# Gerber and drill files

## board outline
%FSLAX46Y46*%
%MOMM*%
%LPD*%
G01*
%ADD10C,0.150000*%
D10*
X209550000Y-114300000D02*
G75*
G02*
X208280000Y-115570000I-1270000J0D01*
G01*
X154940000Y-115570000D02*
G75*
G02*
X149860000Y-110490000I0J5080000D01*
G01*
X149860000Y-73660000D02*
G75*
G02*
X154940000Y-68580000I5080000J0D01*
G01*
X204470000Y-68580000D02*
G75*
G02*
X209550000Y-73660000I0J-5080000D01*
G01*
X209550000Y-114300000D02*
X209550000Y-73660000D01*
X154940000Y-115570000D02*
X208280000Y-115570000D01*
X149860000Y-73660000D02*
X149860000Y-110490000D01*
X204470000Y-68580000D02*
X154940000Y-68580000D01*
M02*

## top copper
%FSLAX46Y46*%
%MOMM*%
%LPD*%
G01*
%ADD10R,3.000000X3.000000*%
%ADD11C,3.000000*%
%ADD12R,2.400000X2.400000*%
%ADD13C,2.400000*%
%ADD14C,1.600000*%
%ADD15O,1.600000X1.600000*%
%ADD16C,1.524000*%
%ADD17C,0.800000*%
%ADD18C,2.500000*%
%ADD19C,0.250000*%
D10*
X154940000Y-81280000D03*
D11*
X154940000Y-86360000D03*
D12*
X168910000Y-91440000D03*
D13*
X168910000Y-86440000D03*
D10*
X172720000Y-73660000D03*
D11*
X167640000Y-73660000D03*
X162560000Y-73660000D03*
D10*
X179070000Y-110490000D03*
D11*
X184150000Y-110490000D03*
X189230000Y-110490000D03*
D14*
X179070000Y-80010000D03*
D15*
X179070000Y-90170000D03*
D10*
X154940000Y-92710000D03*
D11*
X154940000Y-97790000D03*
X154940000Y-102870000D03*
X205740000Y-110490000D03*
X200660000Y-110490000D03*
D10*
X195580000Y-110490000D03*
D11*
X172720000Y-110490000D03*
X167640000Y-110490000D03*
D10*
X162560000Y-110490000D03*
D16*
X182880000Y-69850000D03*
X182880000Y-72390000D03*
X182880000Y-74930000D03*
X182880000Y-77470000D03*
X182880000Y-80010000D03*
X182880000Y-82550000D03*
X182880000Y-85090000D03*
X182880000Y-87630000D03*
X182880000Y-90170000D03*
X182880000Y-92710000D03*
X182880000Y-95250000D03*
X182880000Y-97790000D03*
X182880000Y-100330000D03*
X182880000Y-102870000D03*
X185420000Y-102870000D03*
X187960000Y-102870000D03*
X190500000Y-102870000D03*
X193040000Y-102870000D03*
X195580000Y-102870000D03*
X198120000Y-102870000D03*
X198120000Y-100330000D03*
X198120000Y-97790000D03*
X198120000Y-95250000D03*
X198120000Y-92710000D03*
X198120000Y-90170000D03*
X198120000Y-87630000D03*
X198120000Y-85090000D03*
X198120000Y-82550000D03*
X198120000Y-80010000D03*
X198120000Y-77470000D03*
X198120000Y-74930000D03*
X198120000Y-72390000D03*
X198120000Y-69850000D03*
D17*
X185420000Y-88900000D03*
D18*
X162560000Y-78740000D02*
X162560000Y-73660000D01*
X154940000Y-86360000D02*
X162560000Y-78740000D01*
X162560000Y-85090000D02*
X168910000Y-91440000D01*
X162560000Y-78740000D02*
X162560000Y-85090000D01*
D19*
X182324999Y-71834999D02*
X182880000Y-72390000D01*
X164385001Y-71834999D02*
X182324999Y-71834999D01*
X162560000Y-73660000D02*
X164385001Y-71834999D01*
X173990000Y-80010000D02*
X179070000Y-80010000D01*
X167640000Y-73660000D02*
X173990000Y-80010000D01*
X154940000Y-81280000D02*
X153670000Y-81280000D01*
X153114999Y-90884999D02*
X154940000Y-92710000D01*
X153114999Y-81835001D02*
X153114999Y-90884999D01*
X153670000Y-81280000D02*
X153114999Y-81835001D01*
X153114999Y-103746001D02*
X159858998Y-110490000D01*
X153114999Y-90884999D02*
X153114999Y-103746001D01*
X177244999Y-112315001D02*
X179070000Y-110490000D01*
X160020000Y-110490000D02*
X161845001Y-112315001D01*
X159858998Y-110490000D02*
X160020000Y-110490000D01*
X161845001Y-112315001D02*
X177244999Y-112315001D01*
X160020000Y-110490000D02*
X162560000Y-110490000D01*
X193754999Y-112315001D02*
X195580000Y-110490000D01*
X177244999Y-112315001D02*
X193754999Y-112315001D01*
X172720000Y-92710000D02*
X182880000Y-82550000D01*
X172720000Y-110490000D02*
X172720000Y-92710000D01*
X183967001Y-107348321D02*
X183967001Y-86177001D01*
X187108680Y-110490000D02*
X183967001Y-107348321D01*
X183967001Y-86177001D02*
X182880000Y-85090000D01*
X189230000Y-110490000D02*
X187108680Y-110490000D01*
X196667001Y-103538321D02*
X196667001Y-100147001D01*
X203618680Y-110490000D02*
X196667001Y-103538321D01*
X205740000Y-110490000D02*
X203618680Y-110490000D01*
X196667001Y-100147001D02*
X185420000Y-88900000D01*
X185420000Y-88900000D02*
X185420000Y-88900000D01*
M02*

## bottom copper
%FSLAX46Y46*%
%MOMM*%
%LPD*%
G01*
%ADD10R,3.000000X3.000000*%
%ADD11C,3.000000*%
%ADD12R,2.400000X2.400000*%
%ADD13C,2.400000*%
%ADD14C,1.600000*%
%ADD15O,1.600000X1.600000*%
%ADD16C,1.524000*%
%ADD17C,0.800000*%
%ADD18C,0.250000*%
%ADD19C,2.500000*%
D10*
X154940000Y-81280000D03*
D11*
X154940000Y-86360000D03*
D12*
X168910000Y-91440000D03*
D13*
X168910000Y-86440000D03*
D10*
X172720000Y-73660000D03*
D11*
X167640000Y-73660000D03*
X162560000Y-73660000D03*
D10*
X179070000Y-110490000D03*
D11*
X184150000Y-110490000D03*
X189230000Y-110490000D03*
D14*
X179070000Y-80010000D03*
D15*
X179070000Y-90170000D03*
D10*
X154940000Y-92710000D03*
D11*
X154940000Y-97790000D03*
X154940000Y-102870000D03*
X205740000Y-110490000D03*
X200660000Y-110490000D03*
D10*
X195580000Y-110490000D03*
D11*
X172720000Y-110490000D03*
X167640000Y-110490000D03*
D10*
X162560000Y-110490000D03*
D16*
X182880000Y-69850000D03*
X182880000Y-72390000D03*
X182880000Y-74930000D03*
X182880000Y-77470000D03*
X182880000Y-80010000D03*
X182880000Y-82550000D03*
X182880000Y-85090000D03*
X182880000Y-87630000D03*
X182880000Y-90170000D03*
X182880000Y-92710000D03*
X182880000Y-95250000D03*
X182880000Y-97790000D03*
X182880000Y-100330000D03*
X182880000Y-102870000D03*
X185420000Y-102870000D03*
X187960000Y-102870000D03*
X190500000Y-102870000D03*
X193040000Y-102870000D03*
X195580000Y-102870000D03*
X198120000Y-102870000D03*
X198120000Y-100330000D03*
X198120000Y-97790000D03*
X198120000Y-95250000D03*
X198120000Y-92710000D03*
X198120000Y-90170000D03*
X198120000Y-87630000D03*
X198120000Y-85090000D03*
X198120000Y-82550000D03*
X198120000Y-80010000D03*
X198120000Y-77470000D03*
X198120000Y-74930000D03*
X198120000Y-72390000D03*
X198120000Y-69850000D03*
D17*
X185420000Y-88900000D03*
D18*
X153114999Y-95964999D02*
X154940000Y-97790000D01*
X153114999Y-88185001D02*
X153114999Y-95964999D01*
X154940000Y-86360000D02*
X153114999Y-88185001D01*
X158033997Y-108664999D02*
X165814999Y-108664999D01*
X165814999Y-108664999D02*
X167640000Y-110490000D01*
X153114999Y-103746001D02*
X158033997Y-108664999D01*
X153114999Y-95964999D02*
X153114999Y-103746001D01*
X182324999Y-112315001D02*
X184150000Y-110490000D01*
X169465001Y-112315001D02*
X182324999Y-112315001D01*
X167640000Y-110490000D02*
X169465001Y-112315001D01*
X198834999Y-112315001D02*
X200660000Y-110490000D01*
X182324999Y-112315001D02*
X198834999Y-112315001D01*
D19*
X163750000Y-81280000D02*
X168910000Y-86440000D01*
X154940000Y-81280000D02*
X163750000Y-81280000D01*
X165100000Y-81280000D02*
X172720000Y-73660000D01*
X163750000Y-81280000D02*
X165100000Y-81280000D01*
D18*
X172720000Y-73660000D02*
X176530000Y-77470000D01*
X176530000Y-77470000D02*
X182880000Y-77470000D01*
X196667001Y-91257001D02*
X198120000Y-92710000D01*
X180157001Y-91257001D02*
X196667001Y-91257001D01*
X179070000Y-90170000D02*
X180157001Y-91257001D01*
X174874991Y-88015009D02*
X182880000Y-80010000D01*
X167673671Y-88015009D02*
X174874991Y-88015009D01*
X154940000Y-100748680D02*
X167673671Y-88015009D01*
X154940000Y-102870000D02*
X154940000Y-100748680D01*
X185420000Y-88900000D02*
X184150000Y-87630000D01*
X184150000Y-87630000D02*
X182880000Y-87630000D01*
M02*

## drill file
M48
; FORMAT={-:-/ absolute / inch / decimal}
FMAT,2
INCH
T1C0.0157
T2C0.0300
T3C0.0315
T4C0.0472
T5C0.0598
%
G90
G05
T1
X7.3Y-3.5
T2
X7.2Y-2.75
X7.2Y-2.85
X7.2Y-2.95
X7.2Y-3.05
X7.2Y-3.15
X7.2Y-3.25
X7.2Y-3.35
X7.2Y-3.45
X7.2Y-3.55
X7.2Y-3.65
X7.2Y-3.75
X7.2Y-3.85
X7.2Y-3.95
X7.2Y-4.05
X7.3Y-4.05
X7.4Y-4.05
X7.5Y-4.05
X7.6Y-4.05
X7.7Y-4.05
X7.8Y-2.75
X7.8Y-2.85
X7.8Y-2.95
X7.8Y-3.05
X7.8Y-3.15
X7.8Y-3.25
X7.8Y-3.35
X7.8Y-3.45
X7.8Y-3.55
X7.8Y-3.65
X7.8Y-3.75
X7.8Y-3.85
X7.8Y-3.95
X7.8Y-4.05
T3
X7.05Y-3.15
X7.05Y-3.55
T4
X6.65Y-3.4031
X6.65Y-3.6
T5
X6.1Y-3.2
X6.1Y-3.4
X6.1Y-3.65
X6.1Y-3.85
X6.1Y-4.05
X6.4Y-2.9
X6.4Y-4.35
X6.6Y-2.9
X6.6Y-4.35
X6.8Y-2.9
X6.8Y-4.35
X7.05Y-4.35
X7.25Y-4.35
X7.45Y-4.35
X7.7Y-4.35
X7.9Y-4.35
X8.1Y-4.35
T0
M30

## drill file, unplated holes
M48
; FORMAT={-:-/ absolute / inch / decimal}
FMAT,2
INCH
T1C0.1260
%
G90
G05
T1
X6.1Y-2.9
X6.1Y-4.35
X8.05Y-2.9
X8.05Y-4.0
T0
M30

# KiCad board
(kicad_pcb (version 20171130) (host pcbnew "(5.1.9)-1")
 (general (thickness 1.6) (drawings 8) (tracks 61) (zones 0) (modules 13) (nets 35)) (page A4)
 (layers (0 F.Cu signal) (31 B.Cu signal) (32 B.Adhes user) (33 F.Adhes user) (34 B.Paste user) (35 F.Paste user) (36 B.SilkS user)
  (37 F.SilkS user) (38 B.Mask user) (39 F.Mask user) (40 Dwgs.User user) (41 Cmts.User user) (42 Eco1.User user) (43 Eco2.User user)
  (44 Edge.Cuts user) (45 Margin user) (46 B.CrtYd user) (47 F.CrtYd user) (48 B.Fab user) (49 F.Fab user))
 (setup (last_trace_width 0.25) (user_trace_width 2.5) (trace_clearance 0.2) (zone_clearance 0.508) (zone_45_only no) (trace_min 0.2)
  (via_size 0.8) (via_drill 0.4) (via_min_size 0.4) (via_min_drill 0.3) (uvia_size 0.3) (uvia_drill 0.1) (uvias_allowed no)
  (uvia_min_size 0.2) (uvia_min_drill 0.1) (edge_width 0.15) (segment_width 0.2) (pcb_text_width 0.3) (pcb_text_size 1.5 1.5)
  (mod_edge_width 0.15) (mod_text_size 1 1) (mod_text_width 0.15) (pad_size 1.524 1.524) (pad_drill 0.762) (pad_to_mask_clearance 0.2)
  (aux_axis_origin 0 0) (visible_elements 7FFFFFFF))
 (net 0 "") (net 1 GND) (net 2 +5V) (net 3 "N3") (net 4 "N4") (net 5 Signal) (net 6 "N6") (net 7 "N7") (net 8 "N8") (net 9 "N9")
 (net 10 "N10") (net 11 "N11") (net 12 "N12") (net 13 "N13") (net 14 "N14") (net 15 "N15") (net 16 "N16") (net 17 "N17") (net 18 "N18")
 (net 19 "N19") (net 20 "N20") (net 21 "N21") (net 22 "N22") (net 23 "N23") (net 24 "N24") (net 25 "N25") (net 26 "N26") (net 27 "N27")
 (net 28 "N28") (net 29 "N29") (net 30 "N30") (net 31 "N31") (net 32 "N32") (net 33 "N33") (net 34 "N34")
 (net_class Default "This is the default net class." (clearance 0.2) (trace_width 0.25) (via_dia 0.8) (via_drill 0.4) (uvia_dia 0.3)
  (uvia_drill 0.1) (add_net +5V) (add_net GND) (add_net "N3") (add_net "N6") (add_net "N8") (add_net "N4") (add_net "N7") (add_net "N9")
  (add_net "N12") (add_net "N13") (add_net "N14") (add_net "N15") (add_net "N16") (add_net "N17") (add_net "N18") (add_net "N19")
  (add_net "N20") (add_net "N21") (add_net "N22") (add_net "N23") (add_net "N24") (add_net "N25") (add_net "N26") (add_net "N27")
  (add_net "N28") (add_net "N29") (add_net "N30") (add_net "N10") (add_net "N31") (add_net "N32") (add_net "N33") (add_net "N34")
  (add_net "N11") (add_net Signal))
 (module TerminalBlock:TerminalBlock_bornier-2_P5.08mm (layer F.Cu) (at 154.94 81.28 270)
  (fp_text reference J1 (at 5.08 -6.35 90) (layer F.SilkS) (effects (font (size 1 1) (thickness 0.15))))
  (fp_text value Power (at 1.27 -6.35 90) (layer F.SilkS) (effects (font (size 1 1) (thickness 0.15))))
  (pad 1 thru_hole rect (at 0 0 270) (size 3 3) (drill 1.52) (layers *.Cu *.Mask) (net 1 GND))
  (pad 2 thru_hole circle (at 5.08 0 270) (size 3 3) (drill 1.52) (layers *.Cu *.Mask) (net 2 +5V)))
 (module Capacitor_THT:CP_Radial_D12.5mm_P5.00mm (layer F.Cu) (at 168.91 91.44 90)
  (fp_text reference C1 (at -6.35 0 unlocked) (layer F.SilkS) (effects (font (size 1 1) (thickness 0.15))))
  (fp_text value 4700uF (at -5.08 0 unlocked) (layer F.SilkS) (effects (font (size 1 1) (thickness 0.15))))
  (pad 1 thru_hole rect (at 0 0 90) (size 2.4 2.4) (drill 1.2) (layers *.Cu *.Mask) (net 2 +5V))
  (pad 2 thru_hole circle (at 5 0 90) (size 2.4 2.4) (drill 1.2) (layers *.Cu *.Mask) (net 1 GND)))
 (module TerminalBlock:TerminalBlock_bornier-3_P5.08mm (layer F.Cu) (at 172.72 73.66 180)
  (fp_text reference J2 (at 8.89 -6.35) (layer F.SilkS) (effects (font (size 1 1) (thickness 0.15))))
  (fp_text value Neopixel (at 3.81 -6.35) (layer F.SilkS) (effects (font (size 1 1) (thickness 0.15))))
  (pad 1 thru_hole rect (at 0 0 180) (size 3 3) (drill 1.52) (layers *.Cu *.Mask) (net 1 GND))
  (pad 2 thru_hole circle (at 5.08 0 180) (size 3 3) (drill 1.52) (layers *.Cu *.Mask) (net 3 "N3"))
  (pad 3 thru_hole circle (at 10.16 0 180) (size 3 3) (drill 1.52) (layers *.Cu *.Mask) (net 2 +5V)))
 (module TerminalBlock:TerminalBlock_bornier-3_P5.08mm (layer F.Cu) (at 179.07 110.49)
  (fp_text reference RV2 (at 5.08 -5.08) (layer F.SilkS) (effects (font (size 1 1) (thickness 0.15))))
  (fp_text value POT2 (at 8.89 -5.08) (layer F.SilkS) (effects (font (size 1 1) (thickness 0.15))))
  (pad 1 thru_hole rect (at 0 0) (size 3 3) (drill 1.52) (layers *.Cu *.Mask) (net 1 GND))
  (pad 2 thru_hole circle (at 5.08 0) (size 3 3) (drill 1.52) (layers *.Cu *.Mask) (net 2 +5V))
  (pad 3 thru_hole circle (at 10.16 0) (size 3 3) (drill 1.52) (layers *.Cu *.Mask) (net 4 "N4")))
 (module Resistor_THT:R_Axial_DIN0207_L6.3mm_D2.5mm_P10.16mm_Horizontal (layer F.Cu) (at 179.07 80.01 270)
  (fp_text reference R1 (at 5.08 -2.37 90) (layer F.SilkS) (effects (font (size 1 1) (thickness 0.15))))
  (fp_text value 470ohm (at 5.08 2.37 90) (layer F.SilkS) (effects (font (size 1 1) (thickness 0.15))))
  (pad 1 thru_hole circle (at 0 0 270) (size 1.6 1.6) (drill 0.8) (layers *.Cu *.Mask) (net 3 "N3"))
  (pad 2 thru_hole oval (at 10.16 0 270) (size 1.6 1.6) (drill 0.8) (layers *.Cu *.Mask) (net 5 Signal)))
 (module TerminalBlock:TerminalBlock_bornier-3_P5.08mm (layer F.Cu) (at 154.94 92.71 270)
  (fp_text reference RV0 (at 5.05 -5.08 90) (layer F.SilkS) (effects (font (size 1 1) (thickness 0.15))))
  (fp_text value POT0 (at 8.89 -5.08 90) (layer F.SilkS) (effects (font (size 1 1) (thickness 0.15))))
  (pad 1 thru_hole rect (at 0 0 270) (size 3 3) (drill 1.52) (layers *.Cu *.Mask) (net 1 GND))
  (pad 2 thru_hole circle (at 5.08 0 270) (size 3 3) (drill 1.52) (layers *.Cu *.Mask) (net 2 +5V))
  (pad 3 thru_hole circle (at 10.16 0 270) (size 3 3) (drill 1.52) (layers *.Cu *.Mask) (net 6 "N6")))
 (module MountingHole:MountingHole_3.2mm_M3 (layer F.Cu) (at 204.47 101.6)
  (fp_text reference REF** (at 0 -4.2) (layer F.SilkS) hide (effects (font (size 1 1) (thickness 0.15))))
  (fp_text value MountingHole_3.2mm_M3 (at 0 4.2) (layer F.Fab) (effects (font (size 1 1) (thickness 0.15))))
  (pad 1 np_thru_hole circle (at 0 0) (size 3.2 3.2) (drill 3.2) (layers *.Cu *.Mask)))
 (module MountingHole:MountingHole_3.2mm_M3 (layer F.Cu) (at 154.94 110.49)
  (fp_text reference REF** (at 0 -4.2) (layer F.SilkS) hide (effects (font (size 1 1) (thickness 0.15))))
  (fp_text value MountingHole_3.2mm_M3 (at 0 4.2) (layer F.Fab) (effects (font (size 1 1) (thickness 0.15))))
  (pad 1 np_thru_hole circle (at 0 0) (size 3.2 3.2) (drill 3.2) (layers *.Cu *.Mask)))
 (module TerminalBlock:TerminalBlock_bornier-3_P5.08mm (layer F.Cu) (at 195.58 110.49)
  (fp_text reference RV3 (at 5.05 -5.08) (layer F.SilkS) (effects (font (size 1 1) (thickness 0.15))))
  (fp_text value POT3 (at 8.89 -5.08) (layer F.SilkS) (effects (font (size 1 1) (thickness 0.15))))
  (pad 3 thru_hole circle (at 10.16 0) (size 3 3) (drill 1.52) (layers *.Cu *.Mask) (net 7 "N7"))
  (pad 2 thru_hole circle (at 5.08 0) (size 3 3) (drill 1.52) (layers *.Cu *.Mask) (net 2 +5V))
  (pad 1 thru_hole rect (at 0 0) (size 3 3) (drill 1.52) (layers *.Cu *.Mask) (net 1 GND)))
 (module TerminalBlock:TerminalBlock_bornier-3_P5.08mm (layer F.Cu) (at 162.56 110.49)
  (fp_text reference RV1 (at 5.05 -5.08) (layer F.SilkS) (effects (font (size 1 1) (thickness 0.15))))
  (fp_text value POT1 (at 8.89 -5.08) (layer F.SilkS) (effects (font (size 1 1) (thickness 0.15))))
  (pad 3 thru_hole circle (at 10.16 0) (size 3 3) (drill 1.52) (layers *.Cu *.Mask) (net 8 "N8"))
  (pad 2 thru_hole circle (at 5.08 0) (size 3 3) (drill 1.52) (layers *.Cu *.Mask) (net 2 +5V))
  (pad 1 thru_hole rect (at 0 0) (size 3 3) (drill 1.52) (layers *.Cu *.Mask) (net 1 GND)))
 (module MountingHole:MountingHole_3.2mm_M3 (layer F.Cu) (at 204.47 73.66)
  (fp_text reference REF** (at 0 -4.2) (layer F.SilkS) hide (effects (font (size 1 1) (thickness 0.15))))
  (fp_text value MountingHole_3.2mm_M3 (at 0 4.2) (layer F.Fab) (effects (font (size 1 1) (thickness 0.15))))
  (pad 1 np_thru_hole circle (at 0 0) (size 3.2 3.2) (drill 3.2) (layers *.Cu *.Mask)))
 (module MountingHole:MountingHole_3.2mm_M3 (layer F.Cu) (at 154.94 73.66)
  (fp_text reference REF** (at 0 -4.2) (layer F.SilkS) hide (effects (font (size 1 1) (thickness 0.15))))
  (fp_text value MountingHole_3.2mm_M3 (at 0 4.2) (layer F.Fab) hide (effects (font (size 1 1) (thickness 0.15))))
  (pad 1 np_thru_hole circle (at 0 0) (size 3.2 3.2) (drill 3.2) (layers *.Cu *.Mask)))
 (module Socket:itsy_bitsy (layer F.Cu) (at 182.88 69.85)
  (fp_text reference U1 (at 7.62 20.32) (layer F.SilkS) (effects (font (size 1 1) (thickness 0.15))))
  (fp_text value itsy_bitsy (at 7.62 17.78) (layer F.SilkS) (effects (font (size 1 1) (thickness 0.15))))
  (pad 1 thru_hole circle (at 0 0) (size 1.524 1.524) (drill 0.762) (layers *.Cu *.Mask) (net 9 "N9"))
  (pad 2 thru_hole circle (at 0 2.54) (size 1.524 1.524) (drill 0.762) (layers *.Cu *.Mask) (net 2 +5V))
  (pad 3 thru_hole circle (at 0 5.08) (size 1.524 1.524) (drill 0.762) (layers *.Cu *.Mask) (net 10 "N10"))
  (pad 4 thru_hole circle (at 0 7.62) (size 1.524 1.524) (drill 0.762) (layers *.Cu *.Mask) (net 1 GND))
  (pad 5 thru_hole circle (at 0 10.16) (size 1.524 1.524) (drill 0.762) (layers *.Cu *.Mask) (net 6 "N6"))
  (pad 6 thru_hole circle (at 0 12.7) (size 1.524 1.524) (drill 0.762) (layers *.Cu *.Mask) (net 8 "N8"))
  (pad 7 thru_hole circle (at 0 15.24) (size 1.524 1.524) (drill 0.762) (layers *.Cu *.Mask) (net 4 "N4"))
  (pad 8 thru_hole circle (at 0 17.78) (size 1.524 1.524) (drill 0.762) (layers *.Cu *.Mask) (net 7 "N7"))
  (pad 9 thru_hole circle (at 0 20.32) (size 1.524 1.524) (drill 0.762) (layers *.Cu *.Mask) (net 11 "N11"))
  (pad 10 thru_hole circle (at 0 22.86) (size 1.524 1.524) (drill 0.762) (layers *.Cu *.Mask) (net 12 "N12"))
  (pad 11 thru_hole circle (at 0 25.4) (size 1.524 1.524) (drill 0.762) (layers *.Cu *.Mask) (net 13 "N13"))
  (pad 12 thru_hole circle (at 0 27.94) (size 1.524 1.524) (drill 0.762) (layers *.Cu *.Mask) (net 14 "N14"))
  (pad 13 thru_hole circle (at 0 30.48) (size 1.524 1.524) (drill 0.762) (layers *.Cu *.Mask) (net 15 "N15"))
  (pad 14 thru_hole circle (at 0 33.02) (size 1.524 1.524) (drill 0.762) (layers *.Cu *.Mask) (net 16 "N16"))
  (pad 15 thru_hole circle (at 2.54 33.02) (size 1.524 1.524) (drill 0.762) (layers *.Cu *.Mask) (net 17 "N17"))
  (pad 16 thru_hole circle (at 5.08 33.02) (size 1.524 1.524) (drill 0.762) (layers *.Cu *.Mask) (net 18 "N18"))
  (pad 17 thru_hole circle (at 7.62 33.02) (size 1.524 1.524) (drill 0.762) (layers *.Cu *.Mask) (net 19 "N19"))
  (pad 18 thru_hole circle (at 10.16 33.02) (size 1.524 1.524) (drill 0.762) (layers *.Cu *.Mask) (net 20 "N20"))
  (pad 19 thru_hole circle (at 12.7 33.02) (size 1.524 1.524) (drill 0.762) (layers *.Cu *.Mask) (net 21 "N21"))
  (pad 20 thru_hole circle (at 15.24 33.02) (size 1.524 1.524) (drill 0.762) (layers *.Cu *.Mask) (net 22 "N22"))
  (pad 21 thru_hole circle (at 15.24 30.48) (size 1.524 1.524) (drill 0.762) (layers *.Cu *.Mask) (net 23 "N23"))
  (pad 22 thru_hole circle (at 15.24 27.94) (size 1.524 1.524) (drill 0.762) (layers *.Cu *.Mask) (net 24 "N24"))
  (pad 23 thru_hole circle (at 15.24 25.4) (size 1.524 1.524) (drill 0.762) (layers *.Cu *.Mask) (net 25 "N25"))
  (pad 24 thru_hole circle (at 15.24 22.86) (size 1.524 1.524) (drill 0.762) (layers *.Cu *.Mask) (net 5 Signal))
  (pad 25 thru_hole circle (at 15.24 20.32) (size 1.524 1.524) (drill 0.762) (layers *.Cu *.Mask) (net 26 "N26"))
  (pad 26 thru_hole circle (at 15.24 17.78) (size 1.524 1.524) (drill 0.762) (layers *.Cu *.Mask) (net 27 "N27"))
  (pad 27 thru_hole circle (at 15.24 15.24) (size 1.524 1.524) (drill 0.762) (layers *.Cu *.Mask) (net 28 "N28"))
  (pad 28 thru_hole circle (at 15.24 12.7) (size 1.524 1.524) (drill 0.762) (layers *.Cu *.Mask) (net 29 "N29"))
  (pad 29 thru_hole circle (at 15.24 10.16) (size 1.524 1.524) (drill 0.762) (layers *.Cu *.Mask) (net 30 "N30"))
  (pad 30 thru_hole circle (at 15.24 7.62) (size 1.524 1.524) (drill 0.762) (layers *.Cu *.Mask) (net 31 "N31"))
  (pad 31 thru_hole circle (at 15.24 5.08) (size 1.524 1.524) (drill 0.762) (layers *.Cu *.Mask) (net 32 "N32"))
  (pad 32 thru_hole circle (at 15.24 2.54) (size 1.524 1.524) (drill 0.762) (layers *.Cu *.Mask) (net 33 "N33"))
  (pad 33 thru_hole circle (at 15.24 0) (size 1.524 1.524) (drill 0.762) (layers *.Cu *.Mask) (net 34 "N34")))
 (gr_arc (start 208.28 114.3) (end 208.28 115.57) (angle -90) (layer Edge.Cuts) (width 0.15))
 (gr_arc (start 154.94 110.49) (end 149.86 110.49) (angle -90) (layer Edge.Cuts) (width 0.15))
 (gr_arc (start 154.94 73.66) (end 154.94 68.58) (angle -90) (layer Edge.Cuts) (width 0.15))
 (gr_arc (start 204.47 73.66) (end 209.55 73.66) (angle -90) (layer Edge.Cuts) (width 0.15))
 (gr_line (start 209.55 114.3) (end 209.55 73.66) (layer Edge.Cuts) (width 0.15))
 (gr_line (start 154.94 115.57) (end 208.28 115.57) (layer Edge.Cuts) (width 0.15))
 (gr_line (start 149.86 73.66) (end 149.86 110.49) (layer Edge.Cuts) (width 0.15))
 (gr_line (start 204.47 68.58) (end 154.94 68.58) (layer Edge.Cuts) (width 0.15))
 (segment (start 162.56 78.74) (end 162.56 73.66) (width 2.5) (layer F.Cu) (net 2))
 (segment (start 154.94 86.36) (end 162.56 78.74) (width 2.5) (layer F.Cu) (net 2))
 (segment (start 162.56 85.09) (end 168.91 91.44) (width 2.5) (layer F.Cu) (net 2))
 (segment (start 162.56 78.74) (end 162.56 85.09) (width 2.5) (layer F.Cu) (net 2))
 (segment (start 182.324999 71.834999) (end 182.88 72.39) (width 0.25) (layer F.Cu) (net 2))
 (segment (start 164.385001 71.834999) (end 182.324999 71.834999) (width 0.25) (layer F.Cu) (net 2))
 (segment (start 162.56 73.66) (end 164.385001 71.834999) (width 0.25) (layer F.Cu) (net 2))
 (segment (start 153.114999 95.964999) (end 154.94 97.79) (width 0.25) (layer B.Cu) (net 2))
 (segment (start 153.114999 88.185001) (end 153.114999 95.964999) (width 0.25) (layer B.Cu) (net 2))
 (segment (start 154.94 86.36) (end 153.114999 88.185001) (width 0.25) (layer B.Cu) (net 2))
 (segment (start 158.033997 108.664999) (end 165.814999 108.664999) (width 0.25) (layer B.Cu) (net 2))
 (segment (start 165.814999 108.664999) (end 167.64 110.49) (width 0.25) (layer B.Cu) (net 2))
 (segment (start 153.114999 103.746001) (end 158.033997 108.664999) (width 0.25) (layer B.Cu) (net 2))
 (segment (start 153.114999 95.964999) (end 153.114999 103.746001) (width 0.25) (layer B.Cu) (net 2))
 (segment (start 182.324999 112.315001) (end 184.15 110.49) (width 0.25) (layer B.Cu) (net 2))
 (segment (start 169.465001 112.315001) (end 182.324999 112.315001) (width 0.25) (layer B.Cu) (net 2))
 (segment (start 167.64 110.49) (end 169.465001 112.315001) (width 0.25) (layer B.Cu) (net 2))
 (segment (start 198.834999 112.315001) (end 200.66 110.49) (width 0.25) (layer B.Cu) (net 2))
 (segment (start 182.324999 112.315001) (end 198.834999 112.315001) (width 0.25) (layer B.Cu) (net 2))
 (segment (start 173.99 80.01) (end 179.07 80.01) (width 0.25) (layer F.Cu) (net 3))
 (segment (start 167.64 73.66) (end 173.99 80.01) (width 0.25) (layer F.Cu) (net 3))
 (segment (start 163.75 81.28) (end 168.91 86.44) (width 2.5) (layer B.Cu) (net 1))
 (segment (start 154.94 81.28) (end 163.75 81.28) (width 2.5) (layer B.Cu) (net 1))
 (segment (start 165.1 81.28) (end 172.72 73.66) (width 2.5) (layer B.Cu) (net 1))
 (segment (start 163.75 81.28) (end 165.1 81.28) (width 2.5) (layer B.Cu) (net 1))
 (segment (start 154.94 81.28) (end 153.67 81.28) (width 0.25) (layer F.Cu) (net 1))
 (segment (start 153.114999 90.884999) (end 154.94 92.71) (width 0.25) (layer F.Cu) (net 1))
 (segment (start 153.114999 81.835001) (end 153.114999 90.884999) (width 0.25) (layer F.Cu) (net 1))
 (segment (start 153.67 81.28) (end 153.114999 81.835001) (width 0.25) (layer F.Cu) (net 1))
 (segment (start 153.114999 103.746001) (end 159.858998 110.49) (width 0.25) (layer F.Cu) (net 1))
 (segment (start 153.114999 90.884999) (end 153.114999 103.746001) (width 0.25) (layer F.Cu) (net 1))
 (segment (start 177.244999 112.315001) (end 179.07 110.49) (width 0.25) (layer F.Cu) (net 1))
 (segment (start 160.02 110.49) (end 161.845001 112.315001) (width 0.25) (layer F.Cu) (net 1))
 (segment (start 159.858998 110.49) (end 160.02 110.49) (width 0.25) (layer F.Cu) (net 1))
 (segment (start 161.845001 112.315001) (end 177.244999 112.315001) (width 0.25) (layer F.Cu) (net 1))
 (segment (start 160.02 110.49) (end 162.56 110.49) (width 0.25) (layer F.Cu) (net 1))
 (segment (start 193.754999 112.315001) (end 195.58 110.49) (width 0.25) (layer F.Cu) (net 1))
 (segment (start 177.244999 112.315001) (end 193.754999 112.315001) (width 0.25) (layer F.Cu) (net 1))
 (segment (start 172.72 73.66) (end 176.53 77.47) (width 0.25) (layer B.Cu) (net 1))
 (segment (start 176.53 77.47) (end 182.88 77.47) (width 0.25) (layer B.Cu) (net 1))
 (segment (start 196.667001 91.257001) (end 198.12 92.71) (width 0.25) (layer B.Cu) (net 5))
 (segment (start 180.157001 91.257001) (end 196.667001 91.257001) (width 0.25) (layer B.Cu) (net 5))
 (segment (start 179.07 90.17) (end 180.157001 91.257001) (width 0.25) (layer B.Cu) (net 5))
 (segment (start 174.874991 88.015009) (end 182.88 80.01) (width 0.25) (layer B.Cu) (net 6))
 (segment (start 167.673671 88.015009) (end 174.874991 88.015009) (width 0.25) (layer B.Cu) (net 6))
 (segment (start 154.94 100.74868) (end 167.673671 88.015009) (width 0.25) (layer B.Cu) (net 6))
 (segment (start 154.94 102.87) (end 154.94 100.74868) (width 0.25) (layer B.Cu) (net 6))
 (segment (start 172.72 92.71) (end 182.88 82.55) (width 0.25) (layer F.Cu) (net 8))
 (segment (start 172.72 110.49) (end 172.72 92.71) (width 0.25) (layer F.Cu) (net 8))
 (segment (start 183.967001 107.348321) (end 183.967001 86.177001) (width 0.25) (layer F.Cu) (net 4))
 (segment (start 187.10868 110.49) (end 183.967001 107.348321) (width 0.25) (layer F.Cu) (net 4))
 (segment (start 183.967001 86.177001) (end 182.88 85.09) (width 0.25) (layer F.Cu) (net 4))
 (segment (start 189.23 110.49) (end 187.10868 110.49) (width 0.25) (layer F.Cu) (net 4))
 (segment (start 196.667001 103.538321) (end 196.667001 100.147001) (width 0.25) (layer F.Cu) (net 7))
 (segment (start 203.61868 110.49) (end 196.667001 103.538321) (width 0.25) (layer F.Cu) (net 7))
 (segment (start 205.74 110.49) (end 203.61868 110.49) (width 0.25) (layer F.Cu) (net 7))
 (segment (start 196.667001 100.147001) (end 185.42 88.9) (width 0.25) (layer F.Cu) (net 7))
 (segment (start 185.42 88.9) (end 185.42 88.9) (width 0.25) (layer F.Cu) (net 7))
 (via (at 185.42 88.9) (size 0.8) (drill 0.4) (layers F.Cu B.Cu) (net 7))
 (segment (start 185.42 88.9) (end 184.15 87.63) (width 0.25) (layer B.Cu) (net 7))
 (segment (start 184.15 87.63) (end 182.88 87.63) (width 0.25) (layer B.Cu) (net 7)))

